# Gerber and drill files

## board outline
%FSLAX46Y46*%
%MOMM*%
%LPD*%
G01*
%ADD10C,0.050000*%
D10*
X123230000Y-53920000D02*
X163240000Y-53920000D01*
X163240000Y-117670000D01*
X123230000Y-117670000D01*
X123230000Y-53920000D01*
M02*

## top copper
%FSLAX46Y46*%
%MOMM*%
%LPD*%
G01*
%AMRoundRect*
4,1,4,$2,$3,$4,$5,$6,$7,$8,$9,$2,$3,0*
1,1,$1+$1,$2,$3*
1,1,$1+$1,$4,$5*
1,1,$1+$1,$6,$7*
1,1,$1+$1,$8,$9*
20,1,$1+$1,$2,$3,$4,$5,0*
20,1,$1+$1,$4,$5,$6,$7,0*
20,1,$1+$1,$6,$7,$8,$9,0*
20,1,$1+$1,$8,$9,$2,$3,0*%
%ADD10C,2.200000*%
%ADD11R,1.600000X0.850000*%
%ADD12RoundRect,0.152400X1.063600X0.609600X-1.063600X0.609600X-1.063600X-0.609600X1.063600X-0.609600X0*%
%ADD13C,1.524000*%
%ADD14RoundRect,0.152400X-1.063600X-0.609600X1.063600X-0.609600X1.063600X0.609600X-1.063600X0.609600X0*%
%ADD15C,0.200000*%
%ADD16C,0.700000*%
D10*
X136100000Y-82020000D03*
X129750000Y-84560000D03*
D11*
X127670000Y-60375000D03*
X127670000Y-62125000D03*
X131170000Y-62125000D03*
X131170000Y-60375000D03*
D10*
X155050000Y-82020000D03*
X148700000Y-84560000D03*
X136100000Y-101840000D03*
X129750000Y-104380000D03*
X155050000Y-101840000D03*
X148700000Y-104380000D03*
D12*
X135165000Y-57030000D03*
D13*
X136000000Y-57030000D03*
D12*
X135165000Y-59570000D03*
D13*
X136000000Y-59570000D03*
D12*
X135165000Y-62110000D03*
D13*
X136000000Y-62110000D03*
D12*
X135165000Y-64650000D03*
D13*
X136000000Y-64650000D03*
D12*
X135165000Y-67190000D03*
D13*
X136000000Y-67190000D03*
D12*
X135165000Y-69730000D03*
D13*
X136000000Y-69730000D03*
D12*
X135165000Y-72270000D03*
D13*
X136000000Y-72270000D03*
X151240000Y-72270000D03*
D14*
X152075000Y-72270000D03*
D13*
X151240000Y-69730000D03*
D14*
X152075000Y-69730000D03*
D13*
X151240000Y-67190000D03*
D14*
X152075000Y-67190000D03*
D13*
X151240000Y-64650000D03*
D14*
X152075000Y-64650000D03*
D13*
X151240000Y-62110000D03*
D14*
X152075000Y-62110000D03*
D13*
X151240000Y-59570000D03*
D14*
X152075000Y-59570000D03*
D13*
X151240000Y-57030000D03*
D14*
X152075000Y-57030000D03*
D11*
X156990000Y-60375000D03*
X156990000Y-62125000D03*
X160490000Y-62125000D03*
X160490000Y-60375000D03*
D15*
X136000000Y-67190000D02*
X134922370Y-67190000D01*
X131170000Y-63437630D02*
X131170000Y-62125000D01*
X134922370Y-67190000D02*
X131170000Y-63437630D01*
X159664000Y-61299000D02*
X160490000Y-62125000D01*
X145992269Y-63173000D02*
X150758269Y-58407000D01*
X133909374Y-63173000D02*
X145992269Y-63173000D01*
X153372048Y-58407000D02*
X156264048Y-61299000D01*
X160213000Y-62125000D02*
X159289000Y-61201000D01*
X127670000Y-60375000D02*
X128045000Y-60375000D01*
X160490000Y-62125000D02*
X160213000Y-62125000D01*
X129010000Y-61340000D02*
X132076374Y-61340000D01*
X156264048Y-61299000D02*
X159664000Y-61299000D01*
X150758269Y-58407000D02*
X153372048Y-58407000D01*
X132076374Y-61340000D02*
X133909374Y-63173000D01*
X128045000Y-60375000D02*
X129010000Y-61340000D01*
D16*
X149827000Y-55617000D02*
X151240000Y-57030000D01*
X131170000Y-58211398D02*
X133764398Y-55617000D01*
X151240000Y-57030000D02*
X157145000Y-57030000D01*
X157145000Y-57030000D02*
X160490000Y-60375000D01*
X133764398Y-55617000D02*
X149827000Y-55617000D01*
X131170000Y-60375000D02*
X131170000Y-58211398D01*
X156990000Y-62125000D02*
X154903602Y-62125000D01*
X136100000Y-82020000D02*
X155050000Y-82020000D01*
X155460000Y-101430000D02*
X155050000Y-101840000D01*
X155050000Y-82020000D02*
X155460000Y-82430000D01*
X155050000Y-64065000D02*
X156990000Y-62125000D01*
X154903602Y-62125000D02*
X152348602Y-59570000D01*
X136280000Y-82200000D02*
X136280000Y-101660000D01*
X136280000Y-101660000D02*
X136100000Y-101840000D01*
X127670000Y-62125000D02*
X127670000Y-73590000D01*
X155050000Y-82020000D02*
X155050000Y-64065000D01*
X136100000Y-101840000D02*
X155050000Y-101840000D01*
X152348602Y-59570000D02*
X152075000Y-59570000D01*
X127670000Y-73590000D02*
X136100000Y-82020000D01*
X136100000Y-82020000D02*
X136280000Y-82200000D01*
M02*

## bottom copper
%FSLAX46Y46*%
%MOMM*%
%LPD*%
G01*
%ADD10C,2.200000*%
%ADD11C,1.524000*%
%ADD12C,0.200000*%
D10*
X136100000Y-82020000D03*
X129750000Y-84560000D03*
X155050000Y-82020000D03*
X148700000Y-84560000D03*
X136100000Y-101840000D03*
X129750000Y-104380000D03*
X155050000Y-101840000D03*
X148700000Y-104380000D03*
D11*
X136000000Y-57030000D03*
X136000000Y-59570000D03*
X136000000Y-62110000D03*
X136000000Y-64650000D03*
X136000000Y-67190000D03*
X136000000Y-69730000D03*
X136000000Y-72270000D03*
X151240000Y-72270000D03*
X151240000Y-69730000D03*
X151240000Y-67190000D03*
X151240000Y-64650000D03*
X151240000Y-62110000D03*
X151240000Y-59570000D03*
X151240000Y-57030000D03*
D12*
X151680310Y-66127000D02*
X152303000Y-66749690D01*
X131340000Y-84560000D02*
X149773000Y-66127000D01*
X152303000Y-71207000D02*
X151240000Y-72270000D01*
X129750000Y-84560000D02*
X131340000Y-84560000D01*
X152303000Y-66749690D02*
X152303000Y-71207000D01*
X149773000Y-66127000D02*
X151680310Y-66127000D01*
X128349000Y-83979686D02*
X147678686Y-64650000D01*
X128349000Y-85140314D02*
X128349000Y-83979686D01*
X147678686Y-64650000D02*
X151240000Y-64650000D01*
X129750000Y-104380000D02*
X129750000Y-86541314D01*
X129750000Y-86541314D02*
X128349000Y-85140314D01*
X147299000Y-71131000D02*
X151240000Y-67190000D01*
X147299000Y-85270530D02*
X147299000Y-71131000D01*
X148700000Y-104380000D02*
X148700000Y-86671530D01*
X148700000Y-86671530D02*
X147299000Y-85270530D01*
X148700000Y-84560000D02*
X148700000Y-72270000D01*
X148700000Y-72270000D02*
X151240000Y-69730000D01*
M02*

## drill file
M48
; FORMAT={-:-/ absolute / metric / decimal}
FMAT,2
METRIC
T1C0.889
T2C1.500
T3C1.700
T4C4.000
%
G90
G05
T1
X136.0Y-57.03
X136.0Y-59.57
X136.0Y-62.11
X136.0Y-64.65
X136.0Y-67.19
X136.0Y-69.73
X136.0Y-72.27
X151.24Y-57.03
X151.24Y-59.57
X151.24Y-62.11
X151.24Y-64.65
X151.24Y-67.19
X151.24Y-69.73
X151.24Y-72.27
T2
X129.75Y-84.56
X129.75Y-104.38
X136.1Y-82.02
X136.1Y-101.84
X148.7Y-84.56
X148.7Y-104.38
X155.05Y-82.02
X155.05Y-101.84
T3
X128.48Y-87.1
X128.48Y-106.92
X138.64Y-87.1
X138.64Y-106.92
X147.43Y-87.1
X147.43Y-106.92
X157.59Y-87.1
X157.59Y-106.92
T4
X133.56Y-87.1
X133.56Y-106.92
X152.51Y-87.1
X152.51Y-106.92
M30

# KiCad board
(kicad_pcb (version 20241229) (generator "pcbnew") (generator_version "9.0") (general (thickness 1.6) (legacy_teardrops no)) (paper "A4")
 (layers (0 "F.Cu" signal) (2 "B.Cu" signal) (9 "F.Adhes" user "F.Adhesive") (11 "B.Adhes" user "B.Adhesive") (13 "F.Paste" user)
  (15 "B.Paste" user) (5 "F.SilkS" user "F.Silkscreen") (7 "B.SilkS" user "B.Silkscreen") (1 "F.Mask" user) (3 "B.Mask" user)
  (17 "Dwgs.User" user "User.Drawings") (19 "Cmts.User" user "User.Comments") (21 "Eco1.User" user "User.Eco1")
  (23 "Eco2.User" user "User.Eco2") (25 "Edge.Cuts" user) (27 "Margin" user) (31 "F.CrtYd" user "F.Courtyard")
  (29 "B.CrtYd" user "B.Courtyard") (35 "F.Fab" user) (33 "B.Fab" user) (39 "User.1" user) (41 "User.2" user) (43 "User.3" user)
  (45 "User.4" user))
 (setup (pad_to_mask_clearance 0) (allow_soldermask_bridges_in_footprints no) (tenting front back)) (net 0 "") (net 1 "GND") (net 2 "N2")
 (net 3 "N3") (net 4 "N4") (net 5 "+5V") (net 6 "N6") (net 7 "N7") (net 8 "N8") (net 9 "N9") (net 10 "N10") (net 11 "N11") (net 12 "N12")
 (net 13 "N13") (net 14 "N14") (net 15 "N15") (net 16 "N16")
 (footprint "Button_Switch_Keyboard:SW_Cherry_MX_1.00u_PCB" (layer "F.Cu") (at 136.1 82.02)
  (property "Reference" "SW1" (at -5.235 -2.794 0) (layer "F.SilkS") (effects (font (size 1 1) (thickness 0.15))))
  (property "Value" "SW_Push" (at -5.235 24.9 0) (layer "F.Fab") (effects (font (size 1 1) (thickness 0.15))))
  (pad "" np_thru_hole circle (at -7.62 5.08) (size 1.7 1.7) (drill 1.7) (layers "*.Cu" "*.Mask"))
  (pad "" np_thru_hole circle (at -2.54 5.08) (size 4 4) (drill 4) (layers "*.Cu" "*.Mask"))
  (pad "" np_thru_hole circle (at 2.54 5.08) (size 1.7 1.7) (drill 1.7) (layers "*.Cu" "*.Mask"))
  (pad "1" thru_hole circle (at 0 0) (size 2.2 2.2) (drill 1.5) (layers "*.Cu" "*.Mask") (remove_unused_layers no) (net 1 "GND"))
  (pad "2" thru_hole circle (at -6.35 2.54) (size 2.2 2.2) (drill 1.5) (layers "*.Cu" "*.Mask") (remove_unused_layers no) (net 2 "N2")))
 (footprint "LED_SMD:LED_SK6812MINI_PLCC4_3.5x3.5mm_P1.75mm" (layer "F.Cu") (at 129.42 61.25)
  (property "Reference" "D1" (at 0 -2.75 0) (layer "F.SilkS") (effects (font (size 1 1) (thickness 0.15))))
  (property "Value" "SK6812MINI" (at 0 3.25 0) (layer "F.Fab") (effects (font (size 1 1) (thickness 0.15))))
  (pad "1" smd rect (at -1.75 -0.875) (size 1.6 0.85) (layers "F.Cu" "F.Mask" "F.Paste") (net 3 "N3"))
  (pad "2" smd rect (at -1.75 0.875) (size 1.6 0.85) (layers "F.Cu" "F.Mask" "F.Paste") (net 1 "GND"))
  (pad "3" smd rect (at 1.75 0.875) (size 1.6 0.85) (layers "F.Cu" "F.Mask" "F.Paste") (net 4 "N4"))
  (pad "4" smd rect (at 1.75 -0.875) (size 1.6 0.85) (layers "F.Cu" "F.Mask" "F.Paste") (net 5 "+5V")))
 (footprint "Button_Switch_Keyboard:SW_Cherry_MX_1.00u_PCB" (layer "F.Cu") (at 155.05 82.02)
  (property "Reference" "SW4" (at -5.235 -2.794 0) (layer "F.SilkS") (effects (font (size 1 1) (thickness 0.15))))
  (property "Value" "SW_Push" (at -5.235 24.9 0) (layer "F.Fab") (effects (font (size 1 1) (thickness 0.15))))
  (pad "" np_thru_hole circle (at -7.62 5.08) (size 1.7 1.7) (drill 1.7) (layers "*.Cu" "*.Mask"))
  (pad "" np_thru_hole circle (at -2.54 5.08) (size 4 4) (drill 4) (layers "*.Cu" "*.Mask"))
  (pad "" np_thru_hole circle (at 2.54 5.08) (size 1.7 1.7) (drill 1.7) (layers "*.Cu" "*.Mask"))
  (pad "1" thru_hole circle (at 0 0) (size 2.2 2.2) (drill 1.5) (layers "*.Cu" "*.Mask") (remove_unused_layers no) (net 1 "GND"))
  (pad "2" thru_hole circle (at -6.35 2.54) (size 2.2 2.2) (drill 1.5) (layers "*.Cu" "*.Mask") (remove_unused_layers no) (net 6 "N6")))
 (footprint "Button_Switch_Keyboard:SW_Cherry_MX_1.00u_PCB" (layer "F.Cu") (at 136.1 101.84)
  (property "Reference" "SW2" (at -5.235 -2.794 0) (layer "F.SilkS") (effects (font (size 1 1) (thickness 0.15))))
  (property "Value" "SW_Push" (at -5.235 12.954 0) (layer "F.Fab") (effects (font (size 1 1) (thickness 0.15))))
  (pad "" np_thru_hole circle (at -7.62 5.08) (size 1.7 1.7) (drill 1.7) (layers "*.Cu" "*.Mask"))
  (pad "" np_thru_hole circle (at -2.54 5.08) (size 4 4) (drill 4) (layers "*.Cu" "*.Mask"))
  (pad "" np_thru_hole circle (at 2.54 5.08) (size 1.7 1.7) (drill 1.7) (layers "*.Cu" "*.Mask"))
  (pad "1" thru_hole circle (at 0 0) (size 2.2 2.2) (drill 1.5) (layers "*.Cu" "*.Mask") (remove_unused_layers no) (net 1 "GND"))
  (pad "2" thru_hole circle (at -6.35 2.54) (size 2.2 2.2) (drill 1.5) (layers "*.Cu" "*.Mask") (remove_unused_layers no) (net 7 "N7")))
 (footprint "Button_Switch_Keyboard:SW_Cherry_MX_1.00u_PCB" (layer "F.Cu") (at 155.05 101.84)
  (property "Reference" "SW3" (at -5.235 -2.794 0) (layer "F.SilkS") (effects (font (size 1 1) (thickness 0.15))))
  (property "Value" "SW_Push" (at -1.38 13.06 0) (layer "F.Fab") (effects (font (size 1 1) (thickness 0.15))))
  (pad "" np_thru_hole circle (at -7.62 5.08) (size 1.7 1.7) (drill 1.7) (layers "*.Cu" "*.Mask"))
  (pad "" np_thru_hole circle (at -2.54 5.08) (size 4 4) (drill 4) (layers "*.Cu" "*.Mask"))
  (pad "" np_thru_hole circle (at 2.54 5.08) (size 1.7 1.7) (drill 1.7) (layers "*.Cu" "*.Mask"))
  (pad "1" thru_hole circle (at 0 0) (size 2.2 2.2) (drill 1.5) (layers "*.Cu" "*.Mask") (remove_unused_layers no) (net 1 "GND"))
  (pad "2" thru_hole circle (at -6.35 2.54) (size 2.2 2.2) (drill 1.5) (layers "*.Cu" "*.Mask") (remove_unused_layers no) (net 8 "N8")))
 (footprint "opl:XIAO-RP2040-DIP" (layer "F.Cu") (at 143.62 64.65)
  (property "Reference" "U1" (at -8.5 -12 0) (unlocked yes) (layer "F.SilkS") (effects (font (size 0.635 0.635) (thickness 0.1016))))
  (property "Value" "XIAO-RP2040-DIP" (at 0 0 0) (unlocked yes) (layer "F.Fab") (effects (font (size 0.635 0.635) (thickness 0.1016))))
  (pad "1" smd roundrect (at -8.455 -7.62 180) (size 2.432 1.524) (layers "F.Cu" "F.Mask") (roundrect_rratio 0.1) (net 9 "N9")
   (thermal_bridge_angle 45))
  (pad "1" thru_hole circle (at -7.62 -7.62 180) (size 1.524 1.524) (drill 0.889) (layers "*.Cu" "*.Mask") (remove_unused_layers no)
   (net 9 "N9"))
  (pad "2" smd roundrect (at -8.455 -5.08 180) (size 2.432 1.524) (layers "F.Cu" "F.Mask") (roundrect_rratio 0.1) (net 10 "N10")
   (thermal_bridge_angle 45))
  (pad "2" thru_hole circle (at -7.62 -5.08 180) (size 1.524 1.524) (drill 0.889) (layers "*.Cu" "*.Mask") (remove_unused_layers no)
   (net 10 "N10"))
  (pad "3" smd roundrect (at -8.455 -2.54 180) (size 2.432 1.524) (layers "F.Cu" "F.Mask") (roundrect_rratio 0.1) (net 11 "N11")
   (thermal_bridge_angle 45))
  (pad "3" thru_hole circle (at -7.62 -2.54 180) (size 1.524 1.524) (drill 0.889) (layers "*.Cu" "*.Mask") (remove_unused_layers no)
   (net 11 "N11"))
  (pad "4" smd roundrect (at -8.455 0 180) (size 2.432 1.524) (layers "F.Cu" "F.Mask") (roundrect_rratio 0.1) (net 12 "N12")
   (thermal_bridge_angle 45))
  (pad "4" thru_hole circle (at -7.62 0 180) (size 1.524 1.524) (drill 0.889) (layers "*.Cu" "*.Mask") (remove_unused_layers no)
   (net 12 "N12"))
  (pad "5" smd roundrect (at -8.455 2.54 180) (size 2.432 1.524) (layers "F.Cu" "F.Mask") (roundrect_rratio 0.1) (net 4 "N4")
   (thermal_bridge_angle 45))
  (pad "5" thru_hole circle (at -7.62 2.54 180) (size 1.524 1.524) (drill 0.889) (layers "*.Cu" "*.Mask") (remove_unused_layers no)
   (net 4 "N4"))
  (pad "6" smd roundrect (at -8.455 5.08 180) (size 2.432 1.524) (layers "F.Cu" "F.Mask") (roundrect_rratio 0.1) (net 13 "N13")
   (thermal_bridge_angle 45))
  (pad "6" thru_hole circle (at -7.62 5.08 180) (size 1.524 1.524) (drill 0.889) (layers "*.Cu" "*.Mask") (remove_unused_layers no)
   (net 13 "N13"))
  (pad "7" smd roundrect (at -8.455 7.62 180) (size 2.432 1.524) (layers "F.Cu" "F.Mask") (roundrect_rratio 0.1) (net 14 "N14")
   (thermal_bridge_angle 45))
  (pad "7" thru_hole circle (at -7.62 7.62 180) (size 1.524 1.524) (drill 0.889) (layers "*.Cu" "*.Mask") (remove_unused_layers no)
   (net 14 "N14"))
  (pad "8" thru_hole circle (at 7.62 7.62) (size 1.524 1.524) (drill 0.889) (layers "*.Cu" "*.Mask") (remove_unused_layers no) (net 2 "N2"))
  (pad "8" smd roundrect (at 8.455 7.62) (size 2.432 1.524) (layers "F.Cu" "F.Mask") (roundrect_rratio 0.1) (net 2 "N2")
   (thermal_bridge_angle 45))
  (pad "9" thru_hole circle (at 7.62 5.08) (size 1.524 1.524) (drill 0.889) (layers "*.Cu" "*.Mask") (remove_unused_layers no) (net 6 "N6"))
  (pad "9" smd roundrect (at 8.455 5.08) (size 2.432 1.524) (layers "F.Cu" "F.Mask") (roundrect_rratio 0.1) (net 6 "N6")
   (thermal_bridge_angle 45))
  (pad "10" thru_hole circle (at 7.62 2.54) (size 1.524 1.524) (drill 0.889) (layers "*.Cu" "*.Mask") (remove_unused_layers no) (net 8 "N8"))
  (pad "10" smd roundrect (at 8.455 2.54) (size 2.432 1.524) (layers "F.Cu" "F.Mask") (roundrect_rratio 0.1) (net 8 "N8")
   (thermal_bridge_angle 45))
  (pad "11" thru_hole circle (at 7.62 0) (size 1.524 1.524) (drill 0.889) (layers "*.Cu" "*.Mask") (remove_unused_layers no) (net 7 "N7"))
  (pad "11" smd roundrect (at 8.455 0) (size 2.432 1.524) (layers "F.Cu" "F.Mask") (roundrect_rratio 0.1) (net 7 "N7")
   (thermal_bridge_angle 45))
  (pad "12" thru_hole circle (at 7.62 -2.54) (size 1.524 1.524) (drill 0.889) (layers "*.Cu" "*.Mask") (remove_unused_layers no)
   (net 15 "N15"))
  (pad "12" smd roundrect (at 8.455 -2.54) (size 2.432 1.524) (layers "F.Cu" "F.Mask") (roundrect_rratio 0.1) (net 15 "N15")
   (thermal_bridge_angle 45))
  (pad "13" thru_hole circle (at 7.62 -5.08) (size 1.524 1.524) (drill 0.889) (layers "*.Cu" "*.Mask") (remove_unused_layers no)
   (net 1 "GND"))
  (pad "13" smd roundrect (at 8.455 -5.08) (size 2.432 1.524) (layers "F.Cu" "F.Mask") (roundrect_rratio 0.1) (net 1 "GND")
   (thermal_bridge_angle 45))
  (pad "14" thru_hole circle (at 7.62 -7.62) (size 1.524 1.524) (drill 0.889) (layers "*.Cu" "*.Mask") (remove_unused_layers no)
   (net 5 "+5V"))
  (pad "14" smd roundrect (at 8.455 -7.62) (size 2.432 1.524) (layers "F.Cu" "F.Mask") (roundrect_rratio 0.1) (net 5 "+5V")
   (thermal_bridge_angle 45)))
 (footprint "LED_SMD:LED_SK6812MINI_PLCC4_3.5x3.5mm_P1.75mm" (layer "F.Cu") (at 158.74 61.25)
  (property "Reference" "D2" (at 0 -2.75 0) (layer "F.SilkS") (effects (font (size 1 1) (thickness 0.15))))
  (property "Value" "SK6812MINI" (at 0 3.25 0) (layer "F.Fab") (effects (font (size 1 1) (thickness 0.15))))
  (pad "1" smd rect (at -1.75 -0.875) (size 1.6 0.85) (layers "F.Cu" "F.Mask" "F.Paste") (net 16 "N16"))
  (pad "2" smd rect (at -1.75 0.875) (size 1.6 0.85) (layers "F.Cu" "F.Mask" "F.Paste") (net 1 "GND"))
  (pad "3" smd rect (at 1.75 0.875) (size 1.6 0.85) (layers "F.Cu" "F.Mask" "F.Paste") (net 3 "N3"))
  (pad "4" smd rect (at 1.75 -0.875) (size 1.6 0.85) (layers "F.Cu" "F.Mask" "F.Paste") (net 5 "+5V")))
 (gr_rect (start 123.23 53.92) (end 163.24 117.67) (stroke (width 0.05) (type default)) (fill no) (layer "Edge.Cuts"))
 (segment (start 136 67.19) (end 134.92237 67.19) (width 0.2) (layer "F.Cu") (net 4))
 (segment (start 131.17 63.43763) (end 131.17 62.125) (width 0.2) (layer "F.Cu") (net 4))
 (segment (start 134.92237 67.19) (end 131.17 63.43763) (width 0.2) (layer "F.Cu") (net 4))
 (segment (start 159.664 61.299) (end 160.49 62.125) (width 0.2) (layer "F.Cu") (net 3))
 (segment (start 145.992269 63.173) (end 150.758269 58.407) (width 0.2) (layer "F.Cu") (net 3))
 (segment (start 133.909374 63.173) (end 145.992269 63.173) (width 0.2) (layer "F.Cu") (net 3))
 (segment (start 153.372048 58.407) (end 156.264048 61.299) (width 0.2) (layer "F.Cu") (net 3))
 (segment (start 160.213 62.125) (end 159.289 61.201) (width 0.2) (layer "F.Cu") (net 3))
 (segment (start 127.67 60.375) (end 128.045 60.375) (width 0.2) (layer "F.Cu") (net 3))
 (segment (start 160.49 62.125) (end 160.213 62.125) (width 0.2) (layer "F.Cu") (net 3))
 (segment (start 129.01 61.34) (end 132.076374 61.34) (width 0.2) (layer "F.Cu") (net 3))
 (segment (start 156.264048 61.299) (end 159.664 61.299) (width 0.2) (layer "F.Cu") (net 3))
 (segment (start 150.758269 58.407) (end 153.372048 58.407) (width 0.2) (layer "F.Cu") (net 3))
 (segment (start 132.076374 61.34) (end 133.909374 63.173) (width 0.2) (layer "F.Cu") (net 3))
 (segment (start 128.045 60.375) (end 129.01 61.34) (width 0.2) (layer "F.Cu") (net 3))
 (segment (start 149.827 55.617) (end 151.24 57.03) (width 0.7) (layer "F.Cu") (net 5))
 (segment (start 131.17 58.211398) (end 133.764398 55.617) (width 0.7) (layer "F.Cu") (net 5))
 (segment (start 151.24 57.03) (end 157.145 57.03) (width 0.7) (layer "F.Cu") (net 5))
 (segment (start 157.145 57.03) (end 160.49 60.375) (width 0.7) (layer "F.Cu") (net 5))
 (segment (start 133.764398 55.617) (end 149.827 55.617) (width 0.7) (layer "F.Cu") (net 5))
 (segment (start 131.17 60.375) (end 131.17 58.211398) (width 0.7) (layer "F.Cu") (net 5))
 (segment (start 156.99 62.125) (end 154.903602 62.125) (width 0.7) (layer "F.Cu") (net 1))
 (segment (start 136.1 82.02) (end 155.05 82.02) (width 0.7) (layer "F.Cu") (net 1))
 (segment (start 155.46 101.43) (end 155.05 101.84) (width 0.7) (layer "F.Cu") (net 1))
 (segment (start 155.05 82.02) (end 155.46 82.43) (width 0.7) (layer "F.Cu") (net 1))
 (segment (start 155.05 64.065) (end 156.99 62.125) (width 0.7) (layer "F.Cu") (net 1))
 (segment (start 154.903602 62.125) (end 152.348602 59.57) (width 0.7) (layer "F.Cu") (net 1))
 (segment (start 136.28 82.2) (end 136.28 101.66) (width 0.7) (layer "F.Cu") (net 1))
 (segment (start 136.28 101.66) (end 136.1 101.84) (width 0.7) (layer "F.Cu") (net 1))
 (segment (start 127.67 62.125) (end 127.67 73.59) (width 0.7) (layer "F.Cu") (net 1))
 (segment (start 155.05 82.02) (end 155.05 64.065) (width 0.7) (layer "F.Cu") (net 1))
 (segment (start 136.1 101.84) (end 155.05 101.84) (width 0.7) (layer "F.Cu") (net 1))
 (segment (start 152.348602 59.57) (end 152.075 59.57) (width 0.7) (layer "F.Cu") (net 1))
 (segment (start 127.67 73.59) (end 136.1 82.02) (width 0.7) (layer "F.Cu") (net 1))
 (segment (start 136.1 82.02) (end 136.28 82.2) (width 0.7) (layer "F.Cu") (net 1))
 (segment (start 151.68031 66.127) (end 152.303 66.74969) (width 0.2) (layer "B.Cu") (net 2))
 (segment (start 131.34 84.56) (end 149.773 66.127) (width 0.2) (layer "B.Cu") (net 2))
 (segment (start 152.303 71.207) (end 151.24 72.27) (width 0.2) (layer "B.Cu") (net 2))
 (segment (start 129.75 84.56) (end 131.34 84.56) (width 0.2) (layer "B.Cu") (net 2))
 (segment (start 152.303 66.74969) (end 152.303 71.207) (width 0.2) (layer "B.Cu") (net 2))
 (segment (start 149.773 66.127) (end 151.68031 66.127) (width 0.2) (layer "B.Cu") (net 2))
 (segment (start 128.349 83.979686) (end 147.678686 64.65) (width 0.2) (layer "B.Cu") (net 7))
 (segment (start 128.349 85.140314) (end 128.349 83.979686) (width 0.2) (layer "B.Cu") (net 7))
 (segment (start 147.678686 64.65) (end 151.24 64.65) (width 0.2) (layer "B.Cu") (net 7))
 (segment (start 129.75 104.38) (end 129.75 86.541314) (width 0.2) (layer "B.Cu") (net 7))
 (segment (start 129.75 86.541314) (end 128.349 85.140314) (width 0.2) (layer "B.Cu") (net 7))
 (segment (start 147.299 71.131) (end 151.24 67.19) (width 0.2) (layer "B.Cu") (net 8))
 (segment (start 147.299 85.27053) (end 147.299 71.131) (width 0.2) (layer "B.Cu") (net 8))
 (segment (start 148.7 104.38) (end 148.7 86.67153) (width 0.2) (layer "B.Cu") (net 8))
 (segment (start 148.7 86.67153) (end 147.299 85.27053) (width 0.2) (layer "B.Cu") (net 8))
 (segment (start 148.7 84.56) (end 148.7 72.27) (width 0.2) (layer "B.Cu") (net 6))
 (segment (start 148.7 72.27) (end 151.24 69.73) (width 0.2) (layer "B.Cu") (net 6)))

